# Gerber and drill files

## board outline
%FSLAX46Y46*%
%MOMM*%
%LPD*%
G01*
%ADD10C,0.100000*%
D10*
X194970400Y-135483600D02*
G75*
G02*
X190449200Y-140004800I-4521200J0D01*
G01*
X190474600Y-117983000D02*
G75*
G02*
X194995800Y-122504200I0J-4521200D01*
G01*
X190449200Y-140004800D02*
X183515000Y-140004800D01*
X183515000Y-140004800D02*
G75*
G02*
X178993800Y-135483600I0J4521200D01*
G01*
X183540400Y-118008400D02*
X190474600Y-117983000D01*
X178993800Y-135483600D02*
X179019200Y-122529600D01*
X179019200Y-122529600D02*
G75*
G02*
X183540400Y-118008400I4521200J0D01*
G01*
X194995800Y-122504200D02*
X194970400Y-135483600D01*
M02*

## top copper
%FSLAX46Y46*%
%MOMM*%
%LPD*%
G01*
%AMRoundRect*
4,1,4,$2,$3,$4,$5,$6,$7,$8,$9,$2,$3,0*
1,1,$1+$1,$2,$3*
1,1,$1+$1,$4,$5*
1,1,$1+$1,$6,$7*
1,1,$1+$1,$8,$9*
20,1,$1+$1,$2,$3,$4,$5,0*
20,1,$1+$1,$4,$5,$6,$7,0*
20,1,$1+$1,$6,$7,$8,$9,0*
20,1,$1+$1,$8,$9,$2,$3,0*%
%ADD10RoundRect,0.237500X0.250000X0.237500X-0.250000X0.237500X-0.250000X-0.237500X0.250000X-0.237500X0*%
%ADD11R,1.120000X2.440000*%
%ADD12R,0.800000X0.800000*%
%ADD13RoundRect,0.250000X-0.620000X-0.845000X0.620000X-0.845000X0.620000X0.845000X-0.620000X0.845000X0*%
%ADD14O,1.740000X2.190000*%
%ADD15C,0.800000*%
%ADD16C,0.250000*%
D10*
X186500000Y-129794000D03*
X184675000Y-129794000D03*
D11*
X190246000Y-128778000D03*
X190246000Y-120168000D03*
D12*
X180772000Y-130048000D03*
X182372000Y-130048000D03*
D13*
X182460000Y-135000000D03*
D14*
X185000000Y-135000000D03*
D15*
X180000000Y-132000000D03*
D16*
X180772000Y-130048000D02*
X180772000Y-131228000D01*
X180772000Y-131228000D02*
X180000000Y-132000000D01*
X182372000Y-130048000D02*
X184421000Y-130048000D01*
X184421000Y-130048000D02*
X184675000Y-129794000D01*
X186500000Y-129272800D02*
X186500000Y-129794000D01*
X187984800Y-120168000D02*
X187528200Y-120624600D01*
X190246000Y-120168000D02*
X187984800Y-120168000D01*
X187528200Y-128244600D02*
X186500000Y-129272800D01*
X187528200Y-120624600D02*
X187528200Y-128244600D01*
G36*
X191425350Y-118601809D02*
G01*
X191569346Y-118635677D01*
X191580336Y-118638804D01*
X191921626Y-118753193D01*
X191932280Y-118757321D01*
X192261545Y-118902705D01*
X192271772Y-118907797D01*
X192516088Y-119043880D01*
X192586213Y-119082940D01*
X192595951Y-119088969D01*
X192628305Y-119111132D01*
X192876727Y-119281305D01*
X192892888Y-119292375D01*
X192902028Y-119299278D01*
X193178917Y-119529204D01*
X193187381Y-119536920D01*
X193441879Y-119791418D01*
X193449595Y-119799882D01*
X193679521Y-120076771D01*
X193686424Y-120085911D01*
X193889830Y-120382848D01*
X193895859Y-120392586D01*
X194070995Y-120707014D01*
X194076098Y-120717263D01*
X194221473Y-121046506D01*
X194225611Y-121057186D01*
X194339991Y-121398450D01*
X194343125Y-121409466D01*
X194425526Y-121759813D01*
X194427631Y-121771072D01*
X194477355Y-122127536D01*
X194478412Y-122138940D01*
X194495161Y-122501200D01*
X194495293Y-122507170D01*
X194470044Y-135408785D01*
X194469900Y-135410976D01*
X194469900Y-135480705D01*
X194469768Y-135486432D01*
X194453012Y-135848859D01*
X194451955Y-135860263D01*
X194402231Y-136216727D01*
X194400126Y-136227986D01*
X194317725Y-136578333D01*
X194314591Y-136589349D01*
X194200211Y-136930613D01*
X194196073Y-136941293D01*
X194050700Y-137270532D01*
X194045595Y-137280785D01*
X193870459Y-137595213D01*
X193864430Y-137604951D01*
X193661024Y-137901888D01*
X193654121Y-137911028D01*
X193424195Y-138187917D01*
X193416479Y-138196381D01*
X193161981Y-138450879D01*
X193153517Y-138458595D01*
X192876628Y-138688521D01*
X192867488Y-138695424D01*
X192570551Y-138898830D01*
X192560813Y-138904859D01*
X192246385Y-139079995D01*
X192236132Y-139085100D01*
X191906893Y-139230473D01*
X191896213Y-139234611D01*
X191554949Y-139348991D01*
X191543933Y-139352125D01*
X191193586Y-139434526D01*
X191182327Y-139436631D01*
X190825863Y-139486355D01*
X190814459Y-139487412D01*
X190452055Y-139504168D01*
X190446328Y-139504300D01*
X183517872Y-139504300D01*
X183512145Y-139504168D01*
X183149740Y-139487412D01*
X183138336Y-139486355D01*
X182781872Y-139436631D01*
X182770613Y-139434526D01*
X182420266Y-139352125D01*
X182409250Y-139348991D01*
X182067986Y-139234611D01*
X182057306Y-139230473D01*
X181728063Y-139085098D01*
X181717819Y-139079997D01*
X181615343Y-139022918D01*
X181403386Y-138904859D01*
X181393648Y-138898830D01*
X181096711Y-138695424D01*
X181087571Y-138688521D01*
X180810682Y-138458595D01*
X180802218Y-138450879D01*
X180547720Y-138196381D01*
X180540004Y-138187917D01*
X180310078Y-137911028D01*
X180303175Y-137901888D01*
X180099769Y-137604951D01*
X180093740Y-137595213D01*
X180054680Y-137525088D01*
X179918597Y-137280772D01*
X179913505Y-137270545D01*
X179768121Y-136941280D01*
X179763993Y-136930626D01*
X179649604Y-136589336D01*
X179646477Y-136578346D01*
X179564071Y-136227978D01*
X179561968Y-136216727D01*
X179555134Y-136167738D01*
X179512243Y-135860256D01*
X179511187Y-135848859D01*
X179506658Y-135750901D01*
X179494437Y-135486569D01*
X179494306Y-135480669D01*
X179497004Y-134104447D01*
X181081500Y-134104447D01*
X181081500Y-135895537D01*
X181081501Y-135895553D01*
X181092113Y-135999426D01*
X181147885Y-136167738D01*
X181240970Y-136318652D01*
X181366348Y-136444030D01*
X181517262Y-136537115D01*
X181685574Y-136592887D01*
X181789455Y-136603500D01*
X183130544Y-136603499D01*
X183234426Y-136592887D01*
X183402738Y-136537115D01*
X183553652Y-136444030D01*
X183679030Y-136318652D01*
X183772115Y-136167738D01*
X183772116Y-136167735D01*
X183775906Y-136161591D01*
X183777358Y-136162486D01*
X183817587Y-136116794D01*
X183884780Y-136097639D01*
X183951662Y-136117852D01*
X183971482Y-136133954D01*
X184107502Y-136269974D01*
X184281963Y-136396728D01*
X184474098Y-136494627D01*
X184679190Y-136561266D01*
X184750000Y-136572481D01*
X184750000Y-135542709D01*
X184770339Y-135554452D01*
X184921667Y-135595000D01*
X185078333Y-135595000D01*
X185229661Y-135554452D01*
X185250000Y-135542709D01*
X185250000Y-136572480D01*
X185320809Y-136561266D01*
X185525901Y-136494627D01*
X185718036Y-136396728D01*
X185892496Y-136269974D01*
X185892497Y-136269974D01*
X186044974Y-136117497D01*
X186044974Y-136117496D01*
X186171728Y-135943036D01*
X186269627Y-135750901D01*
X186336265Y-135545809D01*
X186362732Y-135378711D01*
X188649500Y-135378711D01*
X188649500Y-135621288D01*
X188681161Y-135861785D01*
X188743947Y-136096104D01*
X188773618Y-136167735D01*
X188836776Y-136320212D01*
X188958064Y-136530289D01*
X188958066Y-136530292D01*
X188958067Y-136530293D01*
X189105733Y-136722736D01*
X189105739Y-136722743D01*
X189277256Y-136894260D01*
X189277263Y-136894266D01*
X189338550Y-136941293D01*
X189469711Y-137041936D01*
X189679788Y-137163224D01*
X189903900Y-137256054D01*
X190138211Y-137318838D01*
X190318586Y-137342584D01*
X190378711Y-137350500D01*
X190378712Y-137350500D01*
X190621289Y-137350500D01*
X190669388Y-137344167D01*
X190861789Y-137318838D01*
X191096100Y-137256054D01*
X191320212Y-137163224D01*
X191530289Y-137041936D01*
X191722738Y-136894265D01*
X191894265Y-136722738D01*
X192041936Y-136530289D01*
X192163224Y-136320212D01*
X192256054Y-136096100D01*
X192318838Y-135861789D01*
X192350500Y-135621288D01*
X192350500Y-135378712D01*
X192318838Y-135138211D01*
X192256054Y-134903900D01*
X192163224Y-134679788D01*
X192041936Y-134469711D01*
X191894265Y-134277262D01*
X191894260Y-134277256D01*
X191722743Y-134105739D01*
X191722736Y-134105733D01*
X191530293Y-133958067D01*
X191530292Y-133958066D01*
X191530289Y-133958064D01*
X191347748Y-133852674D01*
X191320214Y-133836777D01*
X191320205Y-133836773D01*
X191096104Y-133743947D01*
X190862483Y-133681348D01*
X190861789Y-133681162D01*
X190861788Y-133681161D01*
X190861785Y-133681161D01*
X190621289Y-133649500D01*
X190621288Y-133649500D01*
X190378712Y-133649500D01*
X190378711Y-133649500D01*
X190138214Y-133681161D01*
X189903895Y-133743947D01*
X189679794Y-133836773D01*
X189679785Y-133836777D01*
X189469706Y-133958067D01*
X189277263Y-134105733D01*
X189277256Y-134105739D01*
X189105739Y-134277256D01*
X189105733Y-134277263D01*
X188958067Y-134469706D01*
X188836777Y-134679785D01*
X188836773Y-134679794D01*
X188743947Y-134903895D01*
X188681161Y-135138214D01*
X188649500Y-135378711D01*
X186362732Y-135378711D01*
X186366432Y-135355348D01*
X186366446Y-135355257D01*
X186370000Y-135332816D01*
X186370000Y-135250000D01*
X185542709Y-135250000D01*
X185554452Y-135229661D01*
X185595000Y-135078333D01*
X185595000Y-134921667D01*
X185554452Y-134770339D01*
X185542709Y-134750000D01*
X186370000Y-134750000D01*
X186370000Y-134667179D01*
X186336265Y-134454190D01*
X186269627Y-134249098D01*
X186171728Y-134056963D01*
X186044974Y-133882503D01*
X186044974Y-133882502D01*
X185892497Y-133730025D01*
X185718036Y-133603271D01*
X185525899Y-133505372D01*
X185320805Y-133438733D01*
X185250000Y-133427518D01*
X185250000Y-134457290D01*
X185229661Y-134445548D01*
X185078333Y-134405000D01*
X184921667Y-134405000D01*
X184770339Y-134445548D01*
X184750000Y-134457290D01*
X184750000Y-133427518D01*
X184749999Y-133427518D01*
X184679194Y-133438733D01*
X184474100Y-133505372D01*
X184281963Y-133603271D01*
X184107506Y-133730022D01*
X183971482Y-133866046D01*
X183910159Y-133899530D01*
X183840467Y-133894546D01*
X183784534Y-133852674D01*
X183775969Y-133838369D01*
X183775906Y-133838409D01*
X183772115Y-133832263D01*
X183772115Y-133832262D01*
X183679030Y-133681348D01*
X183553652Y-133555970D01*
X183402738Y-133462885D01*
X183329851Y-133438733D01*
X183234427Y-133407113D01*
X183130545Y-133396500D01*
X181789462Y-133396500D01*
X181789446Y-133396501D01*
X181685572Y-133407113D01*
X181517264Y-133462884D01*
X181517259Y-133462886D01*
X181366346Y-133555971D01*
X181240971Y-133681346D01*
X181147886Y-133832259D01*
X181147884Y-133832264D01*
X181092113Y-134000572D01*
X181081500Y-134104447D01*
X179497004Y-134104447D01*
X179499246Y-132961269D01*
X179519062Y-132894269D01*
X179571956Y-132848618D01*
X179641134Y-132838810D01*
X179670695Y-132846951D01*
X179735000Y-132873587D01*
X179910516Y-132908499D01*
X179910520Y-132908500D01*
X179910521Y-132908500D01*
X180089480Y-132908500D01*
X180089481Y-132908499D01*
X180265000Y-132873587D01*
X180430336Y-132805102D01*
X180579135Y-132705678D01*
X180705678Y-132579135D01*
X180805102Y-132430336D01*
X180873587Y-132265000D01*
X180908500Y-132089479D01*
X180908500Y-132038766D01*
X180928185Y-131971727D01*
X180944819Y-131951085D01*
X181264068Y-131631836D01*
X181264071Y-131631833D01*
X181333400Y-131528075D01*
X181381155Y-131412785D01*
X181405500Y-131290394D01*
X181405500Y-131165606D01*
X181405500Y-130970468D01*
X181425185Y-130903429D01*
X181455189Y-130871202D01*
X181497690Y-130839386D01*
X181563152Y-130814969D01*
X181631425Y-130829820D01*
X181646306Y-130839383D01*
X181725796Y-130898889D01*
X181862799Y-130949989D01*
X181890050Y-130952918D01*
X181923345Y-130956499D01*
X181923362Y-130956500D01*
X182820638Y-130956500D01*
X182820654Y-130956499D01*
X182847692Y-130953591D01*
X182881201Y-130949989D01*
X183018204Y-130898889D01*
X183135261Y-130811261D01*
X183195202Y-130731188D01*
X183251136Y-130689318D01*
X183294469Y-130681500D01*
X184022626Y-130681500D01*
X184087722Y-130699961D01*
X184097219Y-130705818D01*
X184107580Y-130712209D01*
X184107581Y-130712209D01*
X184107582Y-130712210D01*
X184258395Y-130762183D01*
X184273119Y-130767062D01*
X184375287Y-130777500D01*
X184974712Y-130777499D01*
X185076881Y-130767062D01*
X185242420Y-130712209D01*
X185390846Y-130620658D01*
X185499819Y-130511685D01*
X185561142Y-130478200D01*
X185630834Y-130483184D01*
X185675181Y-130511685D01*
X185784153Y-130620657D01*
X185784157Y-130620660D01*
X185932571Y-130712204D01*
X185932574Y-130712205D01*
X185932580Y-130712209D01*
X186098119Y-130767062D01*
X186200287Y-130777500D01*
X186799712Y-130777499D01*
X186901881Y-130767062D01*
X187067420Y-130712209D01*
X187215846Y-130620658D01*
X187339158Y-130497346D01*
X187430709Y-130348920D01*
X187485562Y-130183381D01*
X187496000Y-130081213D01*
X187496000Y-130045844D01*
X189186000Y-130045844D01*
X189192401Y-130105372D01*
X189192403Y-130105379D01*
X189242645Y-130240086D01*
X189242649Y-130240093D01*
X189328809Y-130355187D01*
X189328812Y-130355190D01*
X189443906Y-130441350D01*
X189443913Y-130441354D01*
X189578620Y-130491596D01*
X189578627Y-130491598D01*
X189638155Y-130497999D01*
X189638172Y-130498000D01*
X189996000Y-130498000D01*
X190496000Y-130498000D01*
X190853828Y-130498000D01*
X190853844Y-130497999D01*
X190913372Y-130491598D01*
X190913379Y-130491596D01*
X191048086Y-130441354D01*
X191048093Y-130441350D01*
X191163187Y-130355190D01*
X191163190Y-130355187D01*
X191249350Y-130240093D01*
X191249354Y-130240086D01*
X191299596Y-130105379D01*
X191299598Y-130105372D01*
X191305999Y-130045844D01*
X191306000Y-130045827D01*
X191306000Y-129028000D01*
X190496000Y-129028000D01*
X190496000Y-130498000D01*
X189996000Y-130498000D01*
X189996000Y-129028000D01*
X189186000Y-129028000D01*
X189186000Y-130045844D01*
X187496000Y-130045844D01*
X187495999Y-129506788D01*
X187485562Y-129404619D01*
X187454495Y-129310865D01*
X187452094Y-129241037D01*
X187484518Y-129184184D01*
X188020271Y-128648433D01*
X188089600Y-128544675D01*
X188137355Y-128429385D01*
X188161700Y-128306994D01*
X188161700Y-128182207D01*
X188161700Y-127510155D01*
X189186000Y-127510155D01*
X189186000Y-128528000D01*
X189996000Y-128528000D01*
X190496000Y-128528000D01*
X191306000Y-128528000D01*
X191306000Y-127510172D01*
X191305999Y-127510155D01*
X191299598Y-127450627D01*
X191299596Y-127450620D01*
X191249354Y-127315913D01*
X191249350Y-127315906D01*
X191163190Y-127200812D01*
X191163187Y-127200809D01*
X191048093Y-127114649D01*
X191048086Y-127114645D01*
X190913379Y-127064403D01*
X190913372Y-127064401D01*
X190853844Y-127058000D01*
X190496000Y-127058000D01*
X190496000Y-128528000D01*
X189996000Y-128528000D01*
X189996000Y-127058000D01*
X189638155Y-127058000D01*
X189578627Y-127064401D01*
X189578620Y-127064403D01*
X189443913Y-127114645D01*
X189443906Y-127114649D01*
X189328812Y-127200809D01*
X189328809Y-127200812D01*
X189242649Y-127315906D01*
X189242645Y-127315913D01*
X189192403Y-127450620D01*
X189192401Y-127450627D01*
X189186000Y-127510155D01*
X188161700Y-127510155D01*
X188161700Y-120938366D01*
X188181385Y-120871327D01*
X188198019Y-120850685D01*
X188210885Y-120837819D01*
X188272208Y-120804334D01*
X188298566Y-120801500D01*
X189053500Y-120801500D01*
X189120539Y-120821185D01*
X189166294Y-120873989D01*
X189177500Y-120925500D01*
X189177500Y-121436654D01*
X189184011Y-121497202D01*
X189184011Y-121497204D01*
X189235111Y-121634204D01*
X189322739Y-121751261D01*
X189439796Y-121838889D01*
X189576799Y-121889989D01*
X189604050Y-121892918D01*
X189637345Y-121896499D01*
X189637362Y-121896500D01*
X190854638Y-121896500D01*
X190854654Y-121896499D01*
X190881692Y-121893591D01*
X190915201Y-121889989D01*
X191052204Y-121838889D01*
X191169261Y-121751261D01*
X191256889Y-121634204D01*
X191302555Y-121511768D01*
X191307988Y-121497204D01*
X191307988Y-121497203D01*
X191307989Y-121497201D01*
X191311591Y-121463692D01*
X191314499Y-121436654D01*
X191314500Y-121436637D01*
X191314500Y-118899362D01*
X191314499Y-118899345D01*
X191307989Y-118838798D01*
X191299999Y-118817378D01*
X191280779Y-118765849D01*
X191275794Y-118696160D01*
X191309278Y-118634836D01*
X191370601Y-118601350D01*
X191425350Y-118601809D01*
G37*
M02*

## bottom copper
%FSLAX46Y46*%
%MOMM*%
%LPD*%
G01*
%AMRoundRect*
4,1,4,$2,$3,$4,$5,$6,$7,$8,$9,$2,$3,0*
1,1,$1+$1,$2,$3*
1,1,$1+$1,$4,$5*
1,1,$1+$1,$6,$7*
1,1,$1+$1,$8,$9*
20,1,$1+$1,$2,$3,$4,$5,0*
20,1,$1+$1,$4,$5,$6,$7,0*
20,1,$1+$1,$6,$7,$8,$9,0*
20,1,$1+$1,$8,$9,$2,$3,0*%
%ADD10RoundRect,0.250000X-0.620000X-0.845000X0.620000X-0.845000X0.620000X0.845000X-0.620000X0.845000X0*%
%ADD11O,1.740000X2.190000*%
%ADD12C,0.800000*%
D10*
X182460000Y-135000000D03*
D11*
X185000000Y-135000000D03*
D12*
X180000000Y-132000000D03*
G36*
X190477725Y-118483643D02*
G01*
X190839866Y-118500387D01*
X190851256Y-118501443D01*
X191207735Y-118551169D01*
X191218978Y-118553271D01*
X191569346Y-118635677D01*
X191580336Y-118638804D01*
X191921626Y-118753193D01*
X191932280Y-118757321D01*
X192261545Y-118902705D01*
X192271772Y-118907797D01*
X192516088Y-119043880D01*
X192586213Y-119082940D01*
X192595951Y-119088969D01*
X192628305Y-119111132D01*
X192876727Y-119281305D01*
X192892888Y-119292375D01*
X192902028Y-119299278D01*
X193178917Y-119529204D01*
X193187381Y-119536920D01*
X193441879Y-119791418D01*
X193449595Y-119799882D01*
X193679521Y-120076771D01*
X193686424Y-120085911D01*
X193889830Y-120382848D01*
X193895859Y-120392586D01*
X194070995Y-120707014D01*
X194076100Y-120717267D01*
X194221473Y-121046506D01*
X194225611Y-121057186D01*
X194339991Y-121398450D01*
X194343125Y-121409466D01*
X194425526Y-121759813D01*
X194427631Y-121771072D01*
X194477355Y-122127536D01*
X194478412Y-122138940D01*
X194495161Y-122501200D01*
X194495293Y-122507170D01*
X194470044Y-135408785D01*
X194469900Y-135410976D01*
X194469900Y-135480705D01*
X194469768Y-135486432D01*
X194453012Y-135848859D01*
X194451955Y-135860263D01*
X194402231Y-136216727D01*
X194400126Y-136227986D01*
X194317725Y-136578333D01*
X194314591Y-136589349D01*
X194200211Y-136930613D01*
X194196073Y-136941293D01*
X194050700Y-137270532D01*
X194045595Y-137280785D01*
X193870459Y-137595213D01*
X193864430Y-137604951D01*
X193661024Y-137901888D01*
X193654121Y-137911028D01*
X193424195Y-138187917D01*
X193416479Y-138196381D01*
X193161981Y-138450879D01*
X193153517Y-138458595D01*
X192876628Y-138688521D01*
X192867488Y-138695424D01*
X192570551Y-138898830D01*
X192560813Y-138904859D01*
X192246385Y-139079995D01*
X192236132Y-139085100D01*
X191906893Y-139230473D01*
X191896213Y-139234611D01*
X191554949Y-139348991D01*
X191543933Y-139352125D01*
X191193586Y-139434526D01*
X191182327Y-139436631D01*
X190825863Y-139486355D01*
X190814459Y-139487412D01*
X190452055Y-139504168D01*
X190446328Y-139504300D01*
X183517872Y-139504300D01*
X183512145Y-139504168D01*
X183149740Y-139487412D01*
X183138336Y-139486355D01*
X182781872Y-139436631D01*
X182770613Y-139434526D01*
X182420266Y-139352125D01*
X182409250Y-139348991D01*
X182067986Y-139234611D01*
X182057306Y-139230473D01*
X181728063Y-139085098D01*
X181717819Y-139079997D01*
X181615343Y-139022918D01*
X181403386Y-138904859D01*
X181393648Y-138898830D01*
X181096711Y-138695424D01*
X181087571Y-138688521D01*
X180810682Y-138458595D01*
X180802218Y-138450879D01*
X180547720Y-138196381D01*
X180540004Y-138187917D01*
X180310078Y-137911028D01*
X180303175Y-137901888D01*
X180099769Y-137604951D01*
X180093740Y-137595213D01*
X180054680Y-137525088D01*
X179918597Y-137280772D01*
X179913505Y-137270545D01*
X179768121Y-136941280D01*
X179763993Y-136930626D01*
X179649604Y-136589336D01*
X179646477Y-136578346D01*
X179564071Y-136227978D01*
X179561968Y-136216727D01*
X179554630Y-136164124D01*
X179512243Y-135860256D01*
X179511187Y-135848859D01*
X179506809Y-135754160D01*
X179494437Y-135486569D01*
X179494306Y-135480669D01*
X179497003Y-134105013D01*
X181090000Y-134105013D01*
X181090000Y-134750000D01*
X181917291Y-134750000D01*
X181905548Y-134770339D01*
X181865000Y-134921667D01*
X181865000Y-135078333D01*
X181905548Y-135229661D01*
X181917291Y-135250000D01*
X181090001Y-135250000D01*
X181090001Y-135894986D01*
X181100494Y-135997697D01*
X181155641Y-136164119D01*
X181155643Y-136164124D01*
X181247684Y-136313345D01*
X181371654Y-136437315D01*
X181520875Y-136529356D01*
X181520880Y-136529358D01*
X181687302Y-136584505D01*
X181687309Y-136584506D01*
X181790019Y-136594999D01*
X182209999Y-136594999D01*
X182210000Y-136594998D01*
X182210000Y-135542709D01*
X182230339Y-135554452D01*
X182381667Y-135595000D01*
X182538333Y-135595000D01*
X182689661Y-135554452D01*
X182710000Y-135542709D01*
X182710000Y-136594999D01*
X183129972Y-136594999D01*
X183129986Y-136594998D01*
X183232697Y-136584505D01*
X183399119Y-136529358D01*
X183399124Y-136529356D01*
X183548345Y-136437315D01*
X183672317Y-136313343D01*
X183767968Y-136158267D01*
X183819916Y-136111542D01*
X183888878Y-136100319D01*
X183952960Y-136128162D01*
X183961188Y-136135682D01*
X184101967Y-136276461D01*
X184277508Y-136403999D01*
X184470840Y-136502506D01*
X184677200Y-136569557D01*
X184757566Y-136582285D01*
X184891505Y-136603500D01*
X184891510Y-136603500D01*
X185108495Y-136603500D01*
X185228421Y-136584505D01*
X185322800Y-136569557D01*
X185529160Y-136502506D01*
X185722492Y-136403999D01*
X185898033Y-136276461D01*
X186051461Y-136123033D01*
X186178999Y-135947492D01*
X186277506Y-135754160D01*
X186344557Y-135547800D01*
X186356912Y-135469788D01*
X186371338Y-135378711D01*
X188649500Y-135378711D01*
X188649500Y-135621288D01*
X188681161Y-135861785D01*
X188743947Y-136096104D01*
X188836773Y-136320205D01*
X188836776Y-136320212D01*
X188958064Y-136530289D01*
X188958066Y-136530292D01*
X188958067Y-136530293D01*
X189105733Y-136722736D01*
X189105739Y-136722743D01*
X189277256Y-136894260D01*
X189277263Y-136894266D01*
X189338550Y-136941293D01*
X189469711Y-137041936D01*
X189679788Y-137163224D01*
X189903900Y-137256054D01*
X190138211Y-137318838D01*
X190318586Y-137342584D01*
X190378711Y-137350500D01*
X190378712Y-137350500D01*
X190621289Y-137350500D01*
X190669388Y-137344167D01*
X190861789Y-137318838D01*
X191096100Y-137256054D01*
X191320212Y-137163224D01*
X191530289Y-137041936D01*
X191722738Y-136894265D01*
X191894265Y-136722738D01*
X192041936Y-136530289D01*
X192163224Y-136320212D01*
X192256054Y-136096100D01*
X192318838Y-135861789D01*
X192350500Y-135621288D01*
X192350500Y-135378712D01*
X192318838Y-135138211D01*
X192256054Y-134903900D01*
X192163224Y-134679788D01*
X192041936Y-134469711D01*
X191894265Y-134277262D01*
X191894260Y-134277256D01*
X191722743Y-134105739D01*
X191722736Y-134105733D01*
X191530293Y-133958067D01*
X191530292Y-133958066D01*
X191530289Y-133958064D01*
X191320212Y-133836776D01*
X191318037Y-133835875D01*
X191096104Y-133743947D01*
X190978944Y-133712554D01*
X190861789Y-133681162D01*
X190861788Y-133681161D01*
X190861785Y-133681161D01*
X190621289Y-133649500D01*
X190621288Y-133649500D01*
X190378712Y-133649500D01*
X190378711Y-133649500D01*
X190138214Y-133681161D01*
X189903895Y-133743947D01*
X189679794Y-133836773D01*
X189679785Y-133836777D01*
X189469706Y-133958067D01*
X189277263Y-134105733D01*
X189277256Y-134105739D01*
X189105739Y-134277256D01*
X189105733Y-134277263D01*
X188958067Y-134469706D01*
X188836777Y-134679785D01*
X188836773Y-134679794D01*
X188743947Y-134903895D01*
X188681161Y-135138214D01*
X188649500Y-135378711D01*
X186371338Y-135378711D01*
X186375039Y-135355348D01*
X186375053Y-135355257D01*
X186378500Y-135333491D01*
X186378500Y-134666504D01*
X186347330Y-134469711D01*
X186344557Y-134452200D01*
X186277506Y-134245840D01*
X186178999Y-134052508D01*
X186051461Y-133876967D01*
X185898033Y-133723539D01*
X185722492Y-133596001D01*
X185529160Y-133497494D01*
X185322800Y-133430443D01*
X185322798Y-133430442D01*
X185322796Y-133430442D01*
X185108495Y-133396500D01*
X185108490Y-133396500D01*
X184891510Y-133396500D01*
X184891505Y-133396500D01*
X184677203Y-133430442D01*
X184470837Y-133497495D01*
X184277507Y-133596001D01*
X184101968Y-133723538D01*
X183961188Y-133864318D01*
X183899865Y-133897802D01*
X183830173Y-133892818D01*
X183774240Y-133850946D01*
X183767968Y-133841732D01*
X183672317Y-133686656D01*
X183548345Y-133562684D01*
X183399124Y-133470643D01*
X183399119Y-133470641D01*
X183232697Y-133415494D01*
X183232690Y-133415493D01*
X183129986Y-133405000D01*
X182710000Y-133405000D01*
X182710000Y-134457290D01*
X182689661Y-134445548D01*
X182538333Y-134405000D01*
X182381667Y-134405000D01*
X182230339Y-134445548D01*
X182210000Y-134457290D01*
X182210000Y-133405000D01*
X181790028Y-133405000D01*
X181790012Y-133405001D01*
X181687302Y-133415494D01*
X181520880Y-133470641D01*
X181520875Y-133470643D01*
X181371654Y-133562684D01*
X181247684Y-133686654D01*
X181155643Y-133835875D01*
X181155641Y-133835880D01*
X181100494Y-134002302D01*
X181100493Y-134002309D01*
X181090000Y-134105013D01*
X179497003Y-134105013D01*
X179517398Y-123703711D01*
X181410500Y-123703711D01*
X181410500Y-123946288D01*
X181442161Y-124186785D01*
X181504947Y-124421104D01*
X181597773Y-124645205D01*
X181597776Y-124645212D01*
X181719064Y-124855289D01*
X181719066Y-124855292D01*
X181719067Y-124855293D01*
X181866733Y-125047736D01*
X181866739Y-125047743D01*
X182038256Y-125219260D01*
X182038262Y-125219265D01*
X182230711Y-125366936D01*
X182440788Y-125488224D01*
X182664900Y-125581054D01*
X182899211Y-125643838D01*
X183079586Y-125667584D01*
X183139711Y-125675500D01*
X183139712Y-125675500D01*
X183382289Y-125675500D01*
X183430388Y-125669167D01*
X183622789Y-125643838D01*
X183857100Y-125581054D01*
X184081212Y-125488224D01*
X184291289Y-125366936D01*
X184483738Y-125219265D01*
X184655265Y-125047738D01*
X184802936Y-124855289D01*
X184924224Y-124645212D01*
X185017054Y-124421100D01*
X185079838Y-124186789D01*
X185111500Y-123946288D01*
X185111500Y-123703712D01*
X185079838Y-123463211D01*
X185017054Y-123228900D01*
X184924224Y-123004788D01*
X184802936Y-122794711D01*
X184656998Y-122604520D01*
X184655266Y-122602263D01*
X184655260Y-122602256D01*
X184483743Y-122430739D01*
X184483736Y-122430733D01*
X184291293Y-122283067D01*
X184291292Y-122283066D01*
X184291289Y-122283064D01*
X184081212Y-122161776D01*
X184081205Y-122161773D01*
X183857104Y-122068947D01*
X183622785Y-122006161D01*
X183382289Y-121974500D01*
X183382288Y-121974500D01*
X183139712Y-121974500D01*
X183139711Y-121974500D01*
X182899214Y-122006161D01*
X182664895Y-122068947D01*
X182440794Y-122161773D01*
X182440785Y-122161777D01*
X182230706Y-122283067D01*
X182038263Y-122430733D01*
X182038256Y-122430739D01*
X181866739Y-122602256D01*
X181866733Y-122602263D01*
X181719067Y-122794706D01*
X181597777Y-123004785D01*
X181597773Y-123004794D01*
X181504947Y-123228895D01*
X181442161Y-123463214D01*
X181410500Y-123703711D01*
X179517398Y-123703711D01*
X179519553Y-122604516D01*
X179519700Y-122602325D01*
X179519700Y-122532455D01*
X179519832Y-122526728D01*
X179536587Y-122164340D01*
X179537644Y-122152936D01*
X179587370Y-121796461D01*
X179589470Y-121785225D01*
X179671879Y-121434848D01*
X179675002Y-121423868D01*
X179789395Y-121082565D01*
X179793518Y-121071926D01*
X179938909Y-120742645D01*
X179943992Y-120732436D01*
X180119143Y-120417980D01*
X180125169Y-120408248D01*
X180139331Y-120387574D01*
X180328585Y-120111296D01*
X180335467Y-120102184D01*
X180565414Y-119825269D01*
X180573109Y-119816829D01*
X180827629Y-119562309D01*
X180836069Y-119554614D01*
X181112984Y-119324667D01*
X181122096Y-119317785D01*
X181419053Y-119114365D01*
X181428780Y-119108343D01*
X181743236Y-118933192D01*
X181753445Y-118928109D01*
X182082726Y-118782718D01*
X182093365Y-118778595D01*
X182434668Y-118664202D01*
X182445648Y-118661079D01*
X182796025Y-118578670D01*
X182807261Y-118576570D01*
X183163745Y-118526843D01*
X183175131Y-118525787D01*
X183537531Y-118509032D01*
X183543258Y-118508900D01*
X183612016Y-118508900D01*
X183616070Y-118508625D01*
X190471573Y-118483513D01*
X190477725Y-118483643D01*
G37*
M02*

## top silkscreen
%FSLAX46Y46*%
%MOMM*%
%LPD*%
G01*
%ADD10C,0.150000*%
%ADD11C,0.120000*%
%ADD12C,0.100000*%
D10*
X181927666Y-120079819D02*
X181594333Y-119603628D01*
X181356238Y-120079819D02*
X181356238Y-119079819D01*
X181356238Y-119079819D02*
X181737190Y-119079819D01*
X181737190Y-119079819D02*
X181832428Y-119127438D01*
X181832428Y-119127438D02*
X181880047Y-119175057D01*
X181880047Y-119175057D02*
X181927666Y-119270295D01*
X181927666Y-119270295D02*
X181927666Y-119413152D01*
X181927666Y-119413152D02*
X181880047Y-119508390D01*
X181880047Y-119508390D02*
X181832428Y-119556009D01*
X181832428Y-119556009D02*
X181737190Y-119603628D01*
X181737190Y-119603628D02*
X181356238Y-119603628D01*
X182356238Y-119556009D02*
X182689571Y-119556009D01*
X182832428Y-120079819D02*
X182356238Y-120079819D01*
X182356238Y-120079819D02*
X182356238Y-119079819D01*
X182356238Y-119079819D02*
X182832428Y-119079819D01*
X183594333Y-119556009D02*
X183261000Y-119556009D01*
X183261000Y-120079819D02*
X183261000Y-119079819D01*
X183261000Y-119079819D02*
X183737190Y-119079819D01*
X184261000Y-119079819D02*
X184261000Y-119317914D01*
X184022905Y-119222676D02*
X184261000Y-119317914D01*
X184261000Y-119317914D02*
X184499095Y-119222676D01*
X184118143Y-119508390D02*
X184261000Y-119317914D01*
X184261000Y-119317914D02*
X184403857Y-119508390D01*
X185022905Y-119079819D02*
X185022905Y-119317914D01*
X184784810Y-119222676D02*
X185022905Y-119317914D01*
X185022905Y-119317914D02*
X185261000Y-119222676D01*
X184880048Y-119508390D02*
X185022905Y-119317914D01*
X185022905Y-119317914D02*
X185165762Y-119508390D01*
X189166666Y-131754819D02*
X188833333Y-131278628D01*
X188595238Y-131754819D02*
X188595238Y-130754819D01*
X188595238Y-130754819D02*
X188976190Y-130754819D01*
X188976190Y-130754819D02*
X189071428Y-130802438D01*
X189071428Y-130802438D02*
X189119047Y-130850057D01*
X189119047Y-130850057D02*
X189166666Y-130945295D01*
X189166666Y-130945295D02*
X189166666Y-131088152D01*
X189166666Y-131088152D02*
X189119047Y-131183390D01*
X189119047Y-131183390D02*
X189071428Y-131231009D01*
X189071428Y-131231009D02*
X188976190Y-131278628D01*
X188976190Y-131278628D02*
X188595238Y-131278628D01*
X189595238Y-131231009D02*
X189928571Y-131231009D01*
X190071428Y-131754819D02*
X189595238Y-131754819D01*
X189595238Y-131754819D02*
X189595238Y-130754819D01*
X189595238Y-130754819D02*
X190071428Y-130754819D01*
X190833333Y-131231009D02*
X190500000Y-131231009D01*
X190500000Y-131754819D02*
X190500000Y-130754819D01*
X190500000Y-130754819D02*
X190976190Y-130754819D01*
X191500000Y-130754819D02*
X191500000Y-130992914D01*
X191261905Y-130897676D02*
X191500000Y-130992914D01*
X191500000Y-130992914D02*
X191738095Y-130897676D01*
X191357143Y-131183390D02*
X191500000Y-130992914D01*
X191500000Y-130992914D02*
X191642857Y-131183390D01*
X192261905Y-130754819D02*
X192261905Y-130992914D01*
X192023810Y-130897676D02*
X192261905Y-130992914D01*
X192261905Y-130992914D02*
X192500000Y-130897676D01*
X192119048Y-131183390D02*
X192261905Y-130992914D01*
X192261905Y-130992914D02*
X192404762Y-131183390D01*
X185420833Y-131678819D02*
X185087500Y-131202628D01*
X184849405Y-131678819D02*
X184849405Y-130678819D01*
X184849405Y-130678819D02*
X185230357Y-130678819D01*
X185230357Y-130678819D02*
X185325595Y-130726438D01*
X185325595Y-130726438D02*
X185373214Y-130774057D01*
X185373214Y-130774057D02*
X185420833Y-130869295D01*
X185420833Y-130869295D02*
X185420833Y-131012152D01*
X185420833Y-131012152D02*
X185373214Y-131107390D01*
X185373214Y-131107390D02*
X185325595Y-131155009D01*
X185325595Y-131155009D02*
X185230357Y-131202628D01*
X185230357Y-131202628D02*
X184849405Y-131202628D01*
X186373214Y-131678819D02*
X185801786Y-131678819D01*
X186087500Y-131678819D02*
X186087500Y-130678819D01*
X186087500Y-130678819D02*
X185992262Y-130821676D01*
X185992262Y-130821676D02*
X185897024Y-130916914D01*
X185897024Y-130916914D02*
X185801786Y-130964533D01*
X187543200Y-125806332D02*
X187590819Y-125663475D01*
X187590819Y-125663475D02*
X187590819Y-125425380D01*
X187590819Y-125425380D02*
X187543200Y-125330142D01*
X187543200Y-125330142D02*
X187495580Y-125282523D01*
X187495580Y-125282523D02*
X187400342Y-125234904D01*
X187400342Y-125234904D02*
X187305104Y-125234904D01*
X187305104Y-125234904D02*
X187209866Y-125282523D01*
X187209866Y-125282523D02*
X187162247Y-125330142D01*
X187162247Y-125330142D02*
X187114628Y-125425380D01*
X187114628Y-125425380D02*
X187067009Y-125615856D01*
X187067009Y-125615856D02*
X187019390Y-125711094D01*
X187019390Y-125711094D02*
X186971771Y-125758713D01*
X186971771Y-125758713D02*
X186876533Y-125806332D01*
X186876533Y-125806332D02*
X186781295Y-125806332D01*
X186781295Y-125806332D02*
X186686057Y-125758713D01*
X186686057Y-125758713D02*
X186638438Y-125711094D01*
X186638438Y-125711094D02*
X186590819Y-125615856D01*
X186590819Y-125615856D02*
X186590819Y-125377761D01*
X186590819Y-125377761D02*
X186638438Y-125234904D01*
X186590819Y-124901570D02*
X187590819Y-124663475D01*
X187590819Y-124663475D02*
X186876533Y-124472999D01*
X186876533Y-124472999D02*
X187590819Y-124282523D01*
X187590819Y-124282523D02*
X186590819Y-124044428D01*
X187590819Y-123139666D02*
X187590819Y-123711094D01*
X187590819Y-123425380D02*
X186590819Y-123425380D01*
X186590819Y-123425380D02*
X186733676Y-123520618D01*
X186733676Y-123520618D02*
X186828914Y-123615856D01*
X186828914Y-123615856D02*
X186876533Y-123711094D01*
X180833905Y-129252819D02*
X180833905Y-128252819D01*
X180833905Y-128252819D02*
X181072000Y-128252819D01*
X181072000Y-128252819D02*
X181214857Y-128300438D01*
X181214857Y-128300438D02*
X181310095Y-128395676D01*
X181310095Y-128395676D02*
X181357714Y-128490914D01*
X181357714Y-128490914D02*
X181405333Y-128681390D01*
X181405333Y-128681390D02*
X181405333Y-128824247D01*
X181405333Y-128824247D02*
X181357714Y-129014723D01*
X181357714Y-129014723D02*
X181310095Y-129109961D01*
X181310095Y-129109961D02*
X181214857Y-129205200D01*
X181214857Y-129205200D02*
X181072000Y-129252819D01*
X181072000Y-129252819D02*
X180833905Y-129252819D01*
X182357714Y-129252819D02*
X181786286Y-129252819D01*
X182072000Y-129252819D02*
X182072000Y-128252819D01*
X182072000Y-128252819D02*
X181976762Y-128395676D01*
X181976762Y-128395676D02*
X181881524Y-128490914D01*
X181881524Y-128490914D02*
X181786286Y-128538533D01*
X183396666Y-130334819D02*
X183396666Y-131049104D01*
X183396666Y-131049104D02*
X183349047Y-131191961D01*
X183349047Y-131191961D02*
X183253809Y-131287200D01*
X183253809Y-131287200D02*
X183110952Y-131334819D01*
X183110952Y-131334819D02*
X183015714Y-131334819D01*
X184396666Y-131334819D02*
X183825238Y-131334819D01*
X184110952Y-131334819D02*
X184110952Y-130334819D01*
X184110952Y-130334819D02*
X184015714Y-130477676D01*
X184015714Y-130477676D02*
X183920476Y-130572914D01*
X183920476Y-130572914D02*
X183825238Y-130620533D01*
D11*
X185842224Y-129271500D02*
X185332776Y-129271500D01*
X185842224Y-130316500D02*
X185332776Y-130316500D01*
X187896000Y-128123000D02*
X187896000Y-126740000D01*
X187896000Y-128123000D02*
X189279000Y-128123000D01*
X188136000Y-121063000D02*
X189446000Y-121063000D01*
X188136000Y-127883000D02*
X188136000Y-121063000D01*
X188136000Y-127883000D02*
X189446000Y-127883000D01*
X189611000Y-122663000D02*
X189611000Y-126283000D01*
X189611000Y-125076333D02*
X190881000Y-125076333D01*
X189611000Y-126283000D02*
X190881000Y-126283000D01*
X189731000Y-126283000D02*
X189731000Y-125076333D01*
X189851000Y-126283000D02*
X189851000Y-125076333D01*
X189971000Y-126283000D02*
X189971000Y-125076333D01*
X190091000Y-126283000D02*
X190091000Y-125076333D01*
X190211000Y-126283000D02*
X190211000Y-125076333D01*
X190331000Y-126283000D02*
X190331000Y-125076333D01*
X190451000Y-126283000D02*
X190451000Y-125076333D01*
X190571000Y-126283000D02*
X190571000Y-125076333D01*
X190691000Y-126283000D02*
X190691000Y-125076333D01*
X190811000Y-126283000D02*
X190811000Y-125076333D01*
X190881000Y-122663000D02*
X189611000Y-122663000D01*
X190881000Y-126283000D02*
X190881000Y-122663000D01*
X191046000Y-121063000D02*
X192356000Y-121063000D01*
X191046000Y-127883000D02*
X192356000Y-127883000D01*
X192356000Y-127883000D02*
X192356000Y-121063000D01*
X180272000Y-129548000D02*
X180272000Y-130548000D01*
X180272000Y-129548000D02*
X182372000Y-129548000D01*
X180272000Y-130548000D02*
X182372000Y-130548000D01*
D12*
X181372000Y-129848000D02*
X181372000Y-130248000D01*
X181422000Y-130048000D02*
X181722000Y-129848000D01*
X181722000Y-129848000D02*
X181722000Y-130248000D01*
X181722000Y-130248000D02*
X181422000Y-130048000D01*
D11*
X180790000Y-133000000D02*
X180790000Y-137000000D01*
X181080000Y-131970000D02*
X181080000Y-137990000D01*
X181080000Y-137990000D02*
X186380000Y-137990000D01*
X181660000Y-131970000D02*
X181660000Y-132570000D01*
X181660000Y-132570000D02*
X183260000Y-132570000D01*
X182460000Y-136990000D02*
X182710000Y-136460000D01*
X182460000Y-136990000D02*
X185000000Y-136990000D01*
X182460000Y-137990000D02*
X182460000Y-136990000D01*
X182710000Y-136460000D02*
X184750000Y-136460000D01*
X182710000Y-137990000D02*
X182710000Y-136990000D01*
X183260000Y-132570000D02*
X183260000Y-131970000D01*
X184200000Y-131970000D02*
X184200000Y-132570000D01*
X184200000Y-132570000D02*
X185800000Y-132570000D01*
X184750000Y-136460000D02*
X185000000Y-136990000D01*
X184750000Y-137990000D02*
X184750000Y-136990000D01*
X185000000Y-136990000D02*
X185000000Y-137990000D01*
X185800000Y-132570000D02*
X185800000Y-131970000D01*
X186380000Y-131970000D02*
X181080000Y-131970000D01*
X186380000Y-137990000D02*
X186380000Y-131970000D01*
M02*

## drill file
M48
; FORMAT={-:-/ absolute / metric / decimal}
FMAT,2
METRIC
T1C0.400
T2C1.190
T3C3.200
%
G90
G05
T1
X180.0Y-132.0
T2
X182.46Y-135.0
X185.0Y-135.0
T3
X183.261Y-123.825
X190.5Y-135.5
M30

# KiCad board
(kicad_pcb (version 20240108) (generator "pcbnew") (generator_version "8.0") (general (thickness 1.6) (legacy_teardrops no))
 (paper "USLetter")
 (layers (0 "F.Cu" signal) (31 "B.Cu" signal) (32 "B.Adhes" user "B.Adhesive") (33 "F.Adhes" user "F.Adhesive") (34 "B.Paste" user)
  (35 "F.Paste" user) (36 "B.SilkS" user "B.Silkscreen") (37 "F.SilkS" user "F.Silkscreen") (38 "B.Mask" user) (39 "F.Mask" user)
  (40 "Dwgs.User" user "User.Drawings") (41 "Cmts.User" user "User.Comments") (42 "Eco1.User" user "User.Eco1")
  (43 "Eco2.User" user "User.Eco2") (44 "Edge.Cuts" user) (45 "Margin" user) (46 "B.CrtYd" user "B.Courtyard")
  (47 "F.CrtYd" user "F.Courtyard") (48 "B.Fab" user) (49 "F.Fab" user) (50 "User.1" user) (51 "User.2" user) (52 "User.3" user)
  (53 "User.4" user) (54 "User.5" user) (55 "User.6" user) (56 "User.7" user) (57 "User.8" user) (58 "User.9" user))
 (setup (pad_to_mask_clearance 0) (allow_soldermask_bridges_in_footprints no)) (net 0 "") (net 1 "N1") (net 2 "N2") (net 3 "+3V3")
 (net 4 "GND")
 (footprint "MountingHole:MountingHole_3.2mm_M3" (layer "F.Cu") (at 183.261 123.825)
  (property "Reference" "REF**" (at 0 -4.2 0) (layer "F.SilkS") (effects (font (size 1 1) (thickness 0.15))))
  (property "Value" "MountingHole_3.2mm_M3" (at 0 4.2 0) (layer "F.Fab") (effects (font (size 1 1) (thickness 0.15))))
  (pad "" np_thru_hole circle (at 0 0) (size 3.2 3.2) (drill 3.2) (layers "*.Cu" "*.Mask")))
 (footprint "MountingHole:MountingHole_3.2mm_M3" (layer "F.Cu") (at 190.5 135.5)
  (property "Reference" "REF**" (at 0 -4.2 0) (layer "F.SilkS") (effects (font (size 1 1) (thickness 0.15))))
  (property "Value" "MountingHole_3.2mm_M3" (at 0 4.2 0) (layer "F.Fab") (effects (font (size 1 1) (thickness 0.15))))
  (pad "" np_thru_hole circle (at 0 0) (size 3.2 3.2) (drill 3.2) (layers "*.Cu" "*.Mask")))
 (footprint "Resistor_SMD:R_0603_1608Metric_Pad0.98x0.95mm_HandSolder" (layer "F.Cu") (at 185.5875 129.794 180)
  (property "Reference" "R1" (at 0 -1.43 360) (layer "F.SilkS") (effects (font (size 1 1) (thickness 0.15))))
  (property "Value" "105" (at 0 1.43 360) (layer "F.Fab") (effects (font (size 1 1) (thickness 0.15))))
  (fp_line (start -0.254724 0.5225) (end 0.254724 0.5225) (stroke (width 0.12) (type solid)) (layer "F.SilkS"))
  (fp_line (start -0.254724 -0.5225) (end 0.254724 -0.5225) (stroke (width 0.12) (type solid)) (layer "F.SilkS"))
  (pad "1" smd roundrect (at -0.9125 0 180) (size 0.975 0.95) (layers "F.Cu" "F.Paste" "F.Mask") (roundrect_rratio 0.25) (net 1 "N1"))
  (pad "2" smd roundrect (at 0.9125 0 180) (size 0.975 0.95) (layers "F.Cu" "F.Paste" "F.Mask") (roundrect_rratio 0.25) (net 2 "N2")))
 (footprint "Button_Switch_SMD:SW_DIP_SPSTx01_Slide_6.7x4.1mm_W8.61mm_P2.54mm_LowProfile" (layer "F.Cu") (at 190.246 124.473 90)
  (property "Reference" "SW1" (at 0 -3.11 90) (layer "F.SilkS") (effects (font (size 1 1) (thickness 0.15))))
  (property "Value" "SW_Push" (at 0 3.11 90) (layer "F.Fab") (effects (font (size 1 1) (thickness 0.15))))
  (fp_line (start -3.65 -2.35) (end -2.267 -2.35) (stroke (width 0.12) (type solid)) (layer "F.SilkS"))
  (fp_line (start -3.65 -2.35) (end -3.65 -0.967) (stroke (width 0.12) (type solid)) (layer "F.SilkS"))
  (fp_line (start 3.41 -2.11) (end 3.41 -0.8) (stroke (width 0.12) (type solid)) (layer "F.SilkS"))
  (fp_line (start -3.41 -2.11) (end 3.41 -2.11) (stroke (width 0.12) (type solid)) (layer "F.SilkS"))
  (fp_line (start -3.41 -2.11) (end -3.41 -0.8) (stroke (width 0.12) (type solid)) (layer "F.SilkS"))
  (fp_line (start 1.81 -0.635) (end -1.81 -0.635) (stroke (width 0.12) (type solid)) (layer "F.SilkS"))
  (fp_line (start -0.603333 -0.635) (end -0.603333 0.635) (stroke (width 0.12) (type solid)) (layer "F.SilkS"))
  (fp_line (start -1.81 -0.635) (end -1.81 0.635) (stroke (width 0.12) (type solid)) (layer "F.SilkS"))
  (fp_line (start -1.81 -0.515) (end -0.603333 -0.515) (stroke (width 0.12) (type solid)) (layer "F.SilkS"))
  (fp_line (start -1.81 -0.395) (end -0.603333 -0.395) (stroke (width 0.12) (type solid)) (layer "F.SilkS"))
  (fp_line (start -1.81 -0.275) (end -0.603333 -0.275) (stroke (width 0.12) (type solid)) (layer "F.SilkS"))
  (fp_line (start -1.81 -0.155) (end -0.603333 -0.155) (stroke (width 0.12) (type solid)) (layer "F.SilkS"))
  (fp_line (start -1.81 -0.035) (end -0.603333 -0.035) (stroke (width 0.12) (type solid)) (layer "F.SilkS"))
  (fp_line (start -1.81 0.085) (end -0.603333 0.085) (stroke (width 0.12) (type solid)) (layer "F.SilkS"))
  (fp_line (start -1.81 0.205) (end -0.603333 0.205) (stroke (width 0.12) (type solid)) (layer "F.SilkS"))
  (fp_line (start -1.81 0.325) (end -0.603333 0.325) (stroke (width 0.12) (type solid)) (layer "F.SilkS"))
  (fp_line (start -1.81 0.445) (end -0.603333 0.445) (stroke (width 0.12) (type solid)) (layer "F.SilkS"))
  (fp_line (start -1.81 0.565) (end -0.603333 0.565) (stroke (width 0.12) (type solid)) (layer "F.SilkS"))
  (fp_line (start 1.81 0.635) (end 1.81 -0.635) (stroke (width 0.12) (type solid)) (layer "F.SilkS"))
  (fp_line (start -1.81 0.635) (end 1.81 0.635) (stroke (width 0.12) (type solid)) (layer "F.SilkS"))
  (fp_line (start 3.41 0.8) (end 3.41 2.11) (stroke (width 0.12) (type solid)) (layer "F.SilkS"))
  (fp_line (start -3.41 0.8) (end -3.41 2.11) (stroke (width 0.12) (type solid)) (layer "F.SilkS"))
  (fp_line (start -3.41 2.11) (end 3.41 2.11) (stroke (width 0.12) (type solid)) (layer "F.SilkS"))
  (pad "1" smd rect (at -4.305 0 90) (size 2.44 1.12) (layers "F.Cu" "F.Paste" "F.Mask") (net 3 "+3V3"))
  (pad "2" smd rect (at 4.305 0 90) (size 2.44 1.12) (layers "F.Cu" "F.Paste" "F.Mask") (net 1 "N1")))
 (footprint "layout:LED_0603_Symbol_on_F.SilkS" (layer "F.Cu") (at 181.572 130.048)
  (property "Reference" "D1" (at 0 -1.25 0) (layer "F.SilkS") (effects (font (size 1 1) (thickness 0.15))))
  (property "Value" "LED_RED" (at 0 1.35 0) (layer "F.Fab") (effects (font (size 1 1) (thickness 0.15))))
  (fp_line (start -1.3 -0.5) (end -1.3 0.5) (stroke (width 0.12) (type solid)) (layer "F.SilkS"))
  (fp_line (start -1.3 -0.5) (end 0.8 -0.5) (stroke (width 0.12) (type solid)) (layer "F.SilkS"))
  (fp_line (start -1.3 0.5) (end 0.8 0.5) (stroke (width 0.12) (type solid)) (layer "F.SilkS"))
  (fp_line (start -0.2 -0.2) (end -0.2 0.2) (stroke (width 0.1) (type solid)) (layer "F.SilkS"))
  (fp_line (start -0.15 0) (end 0.15 -0.2) (stroke (width 0.1) (type solid)) (layer "F.SilkS"))
  (fp_line (start 0.15 -0.2) (end 0.15 0.2) (stroke (width 0.1) (type solid)) (layer "F.SilkS"))
  (fp_line (start 0.15 0.2) (end -0.15 0) (stroke (width 0.1) (type solid)) (layer "F.SilkS"))
  (pad "1" smd rect (at -0.8 0 180) (size 0.8 0.8) (layers "F.Cu" "F.Paste" "F.Mask") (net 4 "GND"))
  (pad "2" smd rect (at 0.8 0 180) (size 0.8 0.8) (layers "F.Cu" "F.Paste" "F.Mask") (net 2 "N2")))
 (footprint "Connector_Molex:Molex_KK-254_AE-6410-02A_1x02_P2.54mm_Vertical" (layer "F.Cu") (at 182.46 135)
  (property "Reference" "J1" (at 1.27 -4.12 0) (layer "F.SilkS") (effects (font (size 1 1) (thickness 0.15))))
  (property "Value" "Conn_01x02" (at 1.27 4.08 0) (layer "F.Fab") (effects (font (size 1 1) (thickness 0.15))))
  (fp_line (start -1.67 -2) (end -1.67 2) (stroke (width 0.12) (type solid)) (layer "F.SilkS"))
  (fp_line (start -1.38 -3.03) (end -1.38 2.99) (stroke (width 0.12) (type solid)) (layer "F.SilkS"))
  (fp_line (start -1.38 2.99) (end 3.92 2.99) (stroke (width 0.12) (type solid)) (layer "F.SilkS"))
  (fp_line (start -0.8 -3.03) (end -0.8 -2.43) (stroke (width 0.12) (type solid)) (layer "F.SilkS"))
  (fp_line (start -0.8 -2.43) (end 0.8 -2.43) (stroke (width 0.12) (type solid)) (layer "F.SilkS"))
  (fp_line (start 0 1.99) (end 0.25 1.46) (stroke (width 0.12) (type solid)) (layer "F.SilkS"))
  (fp_line (start 0 1.99) (end 2.54 1.99) (stroke (width 0.12) (type solid)) (layer "F.SilkS"))
  (fp_line (start 0 2.99) (end 0 1.99) (stroke (width 0.12) (type solid)) (layer "F.SilkS"))
  (fp_line (start 0.25 1.46) (end 2.29 1.46) (stroke (width 0.12) (type solid)) (layer "F.SilkS"))
  (fp_line (start 0.25 2.99) (end 0.25 1.99) (stroke (width 0.12) (type solid)) (layer "F.SilkS"))
  (fp_line (start 0.8 -2.43) (end 0.8 -3.03) (stroke (width 0.12) (type solid)) (layer "F.SilkS"))
  (fp_line (start 1.74 -3.03) (end 1.74 -2.43) (stroke (width 0.12) (type solid)) (layer "F.SilkS"))
  (fp_line (start 1.74 -2.43) (end 3.34 -2.43) (stroke (width 0.12) (type solid)) (layer "F.SilkS"))
  (fp_line (start 2.29 1.46) (end 2.54 1.99) (stroke (width 0.12) (type solid)) (layer "F.SilkS"))
  (fp_line (start 2.29 2.99) (end 2.29 1.99) (stroke (width 0.12) (type solid)) (layer "F.SilkS"))
  (fp_line (start 2.54 1.99) (end 2.54 2.99) (stroke (width 0.12) (type solid)) (layer "F.SilkS"))
  (fp_line (start 3.34 -2.43) (end 3.34 -3.03) (stroke (width 0.12) (type solid)) (layer "F.SilkS"))
  (fp_line (start 3.92 -3.03) (end -1.38 -3.03) (stroke (width 0.12) (type solid)) (layer "F.SilkS"))
  (fp_line (start 3.92 2.99) (end 3.92 -3.03) (stroke (width 0.12) (type solid)) (layer "F.SilkS"))
  (pad "1" thru_hole roundrect (at 0 0) (size 1.74 2.19) (drill 1.19) (layers "*.Cu" "*.Mask") (remove_unused_layers no)
   (roundrect_rratio 0.143678) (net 4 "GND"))
  (pad "2" thru_hole oval (at 2.54 0) (size 1.74 2.19) (drill 1.19) (layers "*.Cu" "*.Mask") (remove_unused_layers no) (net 3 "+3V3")))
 (gr_arc (start 194.9704 135.4836) (mid 193.646171 138.680571) (end 190.4492 140.0048) (stroke (width 0.1) (type default))
  (layer "Edge.Cuts"))
 (gr_arc (start 190.4746 117.983) (mid 193.671571 119.307229) (end 194.9958 122.5042) (stroke (width 0.1) (type default))
  (layer "Edge.Cuts"))
 (gr_line (start 190.4492 140.0048) (end 183.515 140.0048) (stroke (width 0.1) (type default)) (layer "Edge.Cuts"))
 (gr_arc (start 183.515 140.0048) (mid 180.318029 138.680571) (end 178.9938 135.4836) (stroke (width 0.1) (type default))
  (layer "Edge.Cuts"))
 (gr_line (start 183.5404 118.0084) (end 190.4746 117.983) (stroke (width 0.1) (type default)) (layer "Edge.Cuts"))
 (gr_line (start 178.9938 135.4836) (end 179.0192 122.5296) (stroke (width 0.1) (type default)) (layer "Edge.Cuts"))
 (gr_arc (start 179.0192 122.5296) (mid 180.343429 119.332629) (end 183.5404 118.0084) (stroke (width 0.1) (type default))
  (layer "Edge.Cuts"))
 (gr_line (start 194.9958 122.5042) (end 194.9704 135.4836) (stroke (width 0.1) (type default)) (layer "Edge.Cuts"))
 (segment (start 180.772 130.048) (end 180.772 131.228) (width 0.25) (layer "F.Cu") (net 4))
 (segment (start 180.772 131.228) (end 180 132) (width 0.25) (layer "F.Cu") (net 4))
 (via (at 180 132) (size 0.8) (drill 0.4) (layers "F.Cu" "B.Cu") (free yes) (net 4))
 (segment (start 182.372 130.048) (end 184.421 130.048) (width 0.25) (layer "F.Cu") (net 2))
 (segment (start 184.421 130.048) (end 184.675 129.794) (width 0.25) (layer "F.Cu") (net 2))
 (segment (start 186.5 129.2728) (end 186.5 129.794) (width 0.25) (layer "F.Cu") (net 1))
 (segment (start 187.9848 120.168) (end 187.5282 120.6246) (width 0.25) (layer "F.Cu") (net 1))
 (segment (start 190.246 120.168) (end 187.9848 120.168) (width 0.25) (layer "F.Cu") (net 1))
 (segment (start 187.5282 128.2446) (end 186.5 129.2728) (width 0.25) (layer "F.Cu") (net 1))
 (segment (start 187.5282 120.6246) (end 187.5282 128.2446) (width 0.25) (layer "F.Cu") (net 1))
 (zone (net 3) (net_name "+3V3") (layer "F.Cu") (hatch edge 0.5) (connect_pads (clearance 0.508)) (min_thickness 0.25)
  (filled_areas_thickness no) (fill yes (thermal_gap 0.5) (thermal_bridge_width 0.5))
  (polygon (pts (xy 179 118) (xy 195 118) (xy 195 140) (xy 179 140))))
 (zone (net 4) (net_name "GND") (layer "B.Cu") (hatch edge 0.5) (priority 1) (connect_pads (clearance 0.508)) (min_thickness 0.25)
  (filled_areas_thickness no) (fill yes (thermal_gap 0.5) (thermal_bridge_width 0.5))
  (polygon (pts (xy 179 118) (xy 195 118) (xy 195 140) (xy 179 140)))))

